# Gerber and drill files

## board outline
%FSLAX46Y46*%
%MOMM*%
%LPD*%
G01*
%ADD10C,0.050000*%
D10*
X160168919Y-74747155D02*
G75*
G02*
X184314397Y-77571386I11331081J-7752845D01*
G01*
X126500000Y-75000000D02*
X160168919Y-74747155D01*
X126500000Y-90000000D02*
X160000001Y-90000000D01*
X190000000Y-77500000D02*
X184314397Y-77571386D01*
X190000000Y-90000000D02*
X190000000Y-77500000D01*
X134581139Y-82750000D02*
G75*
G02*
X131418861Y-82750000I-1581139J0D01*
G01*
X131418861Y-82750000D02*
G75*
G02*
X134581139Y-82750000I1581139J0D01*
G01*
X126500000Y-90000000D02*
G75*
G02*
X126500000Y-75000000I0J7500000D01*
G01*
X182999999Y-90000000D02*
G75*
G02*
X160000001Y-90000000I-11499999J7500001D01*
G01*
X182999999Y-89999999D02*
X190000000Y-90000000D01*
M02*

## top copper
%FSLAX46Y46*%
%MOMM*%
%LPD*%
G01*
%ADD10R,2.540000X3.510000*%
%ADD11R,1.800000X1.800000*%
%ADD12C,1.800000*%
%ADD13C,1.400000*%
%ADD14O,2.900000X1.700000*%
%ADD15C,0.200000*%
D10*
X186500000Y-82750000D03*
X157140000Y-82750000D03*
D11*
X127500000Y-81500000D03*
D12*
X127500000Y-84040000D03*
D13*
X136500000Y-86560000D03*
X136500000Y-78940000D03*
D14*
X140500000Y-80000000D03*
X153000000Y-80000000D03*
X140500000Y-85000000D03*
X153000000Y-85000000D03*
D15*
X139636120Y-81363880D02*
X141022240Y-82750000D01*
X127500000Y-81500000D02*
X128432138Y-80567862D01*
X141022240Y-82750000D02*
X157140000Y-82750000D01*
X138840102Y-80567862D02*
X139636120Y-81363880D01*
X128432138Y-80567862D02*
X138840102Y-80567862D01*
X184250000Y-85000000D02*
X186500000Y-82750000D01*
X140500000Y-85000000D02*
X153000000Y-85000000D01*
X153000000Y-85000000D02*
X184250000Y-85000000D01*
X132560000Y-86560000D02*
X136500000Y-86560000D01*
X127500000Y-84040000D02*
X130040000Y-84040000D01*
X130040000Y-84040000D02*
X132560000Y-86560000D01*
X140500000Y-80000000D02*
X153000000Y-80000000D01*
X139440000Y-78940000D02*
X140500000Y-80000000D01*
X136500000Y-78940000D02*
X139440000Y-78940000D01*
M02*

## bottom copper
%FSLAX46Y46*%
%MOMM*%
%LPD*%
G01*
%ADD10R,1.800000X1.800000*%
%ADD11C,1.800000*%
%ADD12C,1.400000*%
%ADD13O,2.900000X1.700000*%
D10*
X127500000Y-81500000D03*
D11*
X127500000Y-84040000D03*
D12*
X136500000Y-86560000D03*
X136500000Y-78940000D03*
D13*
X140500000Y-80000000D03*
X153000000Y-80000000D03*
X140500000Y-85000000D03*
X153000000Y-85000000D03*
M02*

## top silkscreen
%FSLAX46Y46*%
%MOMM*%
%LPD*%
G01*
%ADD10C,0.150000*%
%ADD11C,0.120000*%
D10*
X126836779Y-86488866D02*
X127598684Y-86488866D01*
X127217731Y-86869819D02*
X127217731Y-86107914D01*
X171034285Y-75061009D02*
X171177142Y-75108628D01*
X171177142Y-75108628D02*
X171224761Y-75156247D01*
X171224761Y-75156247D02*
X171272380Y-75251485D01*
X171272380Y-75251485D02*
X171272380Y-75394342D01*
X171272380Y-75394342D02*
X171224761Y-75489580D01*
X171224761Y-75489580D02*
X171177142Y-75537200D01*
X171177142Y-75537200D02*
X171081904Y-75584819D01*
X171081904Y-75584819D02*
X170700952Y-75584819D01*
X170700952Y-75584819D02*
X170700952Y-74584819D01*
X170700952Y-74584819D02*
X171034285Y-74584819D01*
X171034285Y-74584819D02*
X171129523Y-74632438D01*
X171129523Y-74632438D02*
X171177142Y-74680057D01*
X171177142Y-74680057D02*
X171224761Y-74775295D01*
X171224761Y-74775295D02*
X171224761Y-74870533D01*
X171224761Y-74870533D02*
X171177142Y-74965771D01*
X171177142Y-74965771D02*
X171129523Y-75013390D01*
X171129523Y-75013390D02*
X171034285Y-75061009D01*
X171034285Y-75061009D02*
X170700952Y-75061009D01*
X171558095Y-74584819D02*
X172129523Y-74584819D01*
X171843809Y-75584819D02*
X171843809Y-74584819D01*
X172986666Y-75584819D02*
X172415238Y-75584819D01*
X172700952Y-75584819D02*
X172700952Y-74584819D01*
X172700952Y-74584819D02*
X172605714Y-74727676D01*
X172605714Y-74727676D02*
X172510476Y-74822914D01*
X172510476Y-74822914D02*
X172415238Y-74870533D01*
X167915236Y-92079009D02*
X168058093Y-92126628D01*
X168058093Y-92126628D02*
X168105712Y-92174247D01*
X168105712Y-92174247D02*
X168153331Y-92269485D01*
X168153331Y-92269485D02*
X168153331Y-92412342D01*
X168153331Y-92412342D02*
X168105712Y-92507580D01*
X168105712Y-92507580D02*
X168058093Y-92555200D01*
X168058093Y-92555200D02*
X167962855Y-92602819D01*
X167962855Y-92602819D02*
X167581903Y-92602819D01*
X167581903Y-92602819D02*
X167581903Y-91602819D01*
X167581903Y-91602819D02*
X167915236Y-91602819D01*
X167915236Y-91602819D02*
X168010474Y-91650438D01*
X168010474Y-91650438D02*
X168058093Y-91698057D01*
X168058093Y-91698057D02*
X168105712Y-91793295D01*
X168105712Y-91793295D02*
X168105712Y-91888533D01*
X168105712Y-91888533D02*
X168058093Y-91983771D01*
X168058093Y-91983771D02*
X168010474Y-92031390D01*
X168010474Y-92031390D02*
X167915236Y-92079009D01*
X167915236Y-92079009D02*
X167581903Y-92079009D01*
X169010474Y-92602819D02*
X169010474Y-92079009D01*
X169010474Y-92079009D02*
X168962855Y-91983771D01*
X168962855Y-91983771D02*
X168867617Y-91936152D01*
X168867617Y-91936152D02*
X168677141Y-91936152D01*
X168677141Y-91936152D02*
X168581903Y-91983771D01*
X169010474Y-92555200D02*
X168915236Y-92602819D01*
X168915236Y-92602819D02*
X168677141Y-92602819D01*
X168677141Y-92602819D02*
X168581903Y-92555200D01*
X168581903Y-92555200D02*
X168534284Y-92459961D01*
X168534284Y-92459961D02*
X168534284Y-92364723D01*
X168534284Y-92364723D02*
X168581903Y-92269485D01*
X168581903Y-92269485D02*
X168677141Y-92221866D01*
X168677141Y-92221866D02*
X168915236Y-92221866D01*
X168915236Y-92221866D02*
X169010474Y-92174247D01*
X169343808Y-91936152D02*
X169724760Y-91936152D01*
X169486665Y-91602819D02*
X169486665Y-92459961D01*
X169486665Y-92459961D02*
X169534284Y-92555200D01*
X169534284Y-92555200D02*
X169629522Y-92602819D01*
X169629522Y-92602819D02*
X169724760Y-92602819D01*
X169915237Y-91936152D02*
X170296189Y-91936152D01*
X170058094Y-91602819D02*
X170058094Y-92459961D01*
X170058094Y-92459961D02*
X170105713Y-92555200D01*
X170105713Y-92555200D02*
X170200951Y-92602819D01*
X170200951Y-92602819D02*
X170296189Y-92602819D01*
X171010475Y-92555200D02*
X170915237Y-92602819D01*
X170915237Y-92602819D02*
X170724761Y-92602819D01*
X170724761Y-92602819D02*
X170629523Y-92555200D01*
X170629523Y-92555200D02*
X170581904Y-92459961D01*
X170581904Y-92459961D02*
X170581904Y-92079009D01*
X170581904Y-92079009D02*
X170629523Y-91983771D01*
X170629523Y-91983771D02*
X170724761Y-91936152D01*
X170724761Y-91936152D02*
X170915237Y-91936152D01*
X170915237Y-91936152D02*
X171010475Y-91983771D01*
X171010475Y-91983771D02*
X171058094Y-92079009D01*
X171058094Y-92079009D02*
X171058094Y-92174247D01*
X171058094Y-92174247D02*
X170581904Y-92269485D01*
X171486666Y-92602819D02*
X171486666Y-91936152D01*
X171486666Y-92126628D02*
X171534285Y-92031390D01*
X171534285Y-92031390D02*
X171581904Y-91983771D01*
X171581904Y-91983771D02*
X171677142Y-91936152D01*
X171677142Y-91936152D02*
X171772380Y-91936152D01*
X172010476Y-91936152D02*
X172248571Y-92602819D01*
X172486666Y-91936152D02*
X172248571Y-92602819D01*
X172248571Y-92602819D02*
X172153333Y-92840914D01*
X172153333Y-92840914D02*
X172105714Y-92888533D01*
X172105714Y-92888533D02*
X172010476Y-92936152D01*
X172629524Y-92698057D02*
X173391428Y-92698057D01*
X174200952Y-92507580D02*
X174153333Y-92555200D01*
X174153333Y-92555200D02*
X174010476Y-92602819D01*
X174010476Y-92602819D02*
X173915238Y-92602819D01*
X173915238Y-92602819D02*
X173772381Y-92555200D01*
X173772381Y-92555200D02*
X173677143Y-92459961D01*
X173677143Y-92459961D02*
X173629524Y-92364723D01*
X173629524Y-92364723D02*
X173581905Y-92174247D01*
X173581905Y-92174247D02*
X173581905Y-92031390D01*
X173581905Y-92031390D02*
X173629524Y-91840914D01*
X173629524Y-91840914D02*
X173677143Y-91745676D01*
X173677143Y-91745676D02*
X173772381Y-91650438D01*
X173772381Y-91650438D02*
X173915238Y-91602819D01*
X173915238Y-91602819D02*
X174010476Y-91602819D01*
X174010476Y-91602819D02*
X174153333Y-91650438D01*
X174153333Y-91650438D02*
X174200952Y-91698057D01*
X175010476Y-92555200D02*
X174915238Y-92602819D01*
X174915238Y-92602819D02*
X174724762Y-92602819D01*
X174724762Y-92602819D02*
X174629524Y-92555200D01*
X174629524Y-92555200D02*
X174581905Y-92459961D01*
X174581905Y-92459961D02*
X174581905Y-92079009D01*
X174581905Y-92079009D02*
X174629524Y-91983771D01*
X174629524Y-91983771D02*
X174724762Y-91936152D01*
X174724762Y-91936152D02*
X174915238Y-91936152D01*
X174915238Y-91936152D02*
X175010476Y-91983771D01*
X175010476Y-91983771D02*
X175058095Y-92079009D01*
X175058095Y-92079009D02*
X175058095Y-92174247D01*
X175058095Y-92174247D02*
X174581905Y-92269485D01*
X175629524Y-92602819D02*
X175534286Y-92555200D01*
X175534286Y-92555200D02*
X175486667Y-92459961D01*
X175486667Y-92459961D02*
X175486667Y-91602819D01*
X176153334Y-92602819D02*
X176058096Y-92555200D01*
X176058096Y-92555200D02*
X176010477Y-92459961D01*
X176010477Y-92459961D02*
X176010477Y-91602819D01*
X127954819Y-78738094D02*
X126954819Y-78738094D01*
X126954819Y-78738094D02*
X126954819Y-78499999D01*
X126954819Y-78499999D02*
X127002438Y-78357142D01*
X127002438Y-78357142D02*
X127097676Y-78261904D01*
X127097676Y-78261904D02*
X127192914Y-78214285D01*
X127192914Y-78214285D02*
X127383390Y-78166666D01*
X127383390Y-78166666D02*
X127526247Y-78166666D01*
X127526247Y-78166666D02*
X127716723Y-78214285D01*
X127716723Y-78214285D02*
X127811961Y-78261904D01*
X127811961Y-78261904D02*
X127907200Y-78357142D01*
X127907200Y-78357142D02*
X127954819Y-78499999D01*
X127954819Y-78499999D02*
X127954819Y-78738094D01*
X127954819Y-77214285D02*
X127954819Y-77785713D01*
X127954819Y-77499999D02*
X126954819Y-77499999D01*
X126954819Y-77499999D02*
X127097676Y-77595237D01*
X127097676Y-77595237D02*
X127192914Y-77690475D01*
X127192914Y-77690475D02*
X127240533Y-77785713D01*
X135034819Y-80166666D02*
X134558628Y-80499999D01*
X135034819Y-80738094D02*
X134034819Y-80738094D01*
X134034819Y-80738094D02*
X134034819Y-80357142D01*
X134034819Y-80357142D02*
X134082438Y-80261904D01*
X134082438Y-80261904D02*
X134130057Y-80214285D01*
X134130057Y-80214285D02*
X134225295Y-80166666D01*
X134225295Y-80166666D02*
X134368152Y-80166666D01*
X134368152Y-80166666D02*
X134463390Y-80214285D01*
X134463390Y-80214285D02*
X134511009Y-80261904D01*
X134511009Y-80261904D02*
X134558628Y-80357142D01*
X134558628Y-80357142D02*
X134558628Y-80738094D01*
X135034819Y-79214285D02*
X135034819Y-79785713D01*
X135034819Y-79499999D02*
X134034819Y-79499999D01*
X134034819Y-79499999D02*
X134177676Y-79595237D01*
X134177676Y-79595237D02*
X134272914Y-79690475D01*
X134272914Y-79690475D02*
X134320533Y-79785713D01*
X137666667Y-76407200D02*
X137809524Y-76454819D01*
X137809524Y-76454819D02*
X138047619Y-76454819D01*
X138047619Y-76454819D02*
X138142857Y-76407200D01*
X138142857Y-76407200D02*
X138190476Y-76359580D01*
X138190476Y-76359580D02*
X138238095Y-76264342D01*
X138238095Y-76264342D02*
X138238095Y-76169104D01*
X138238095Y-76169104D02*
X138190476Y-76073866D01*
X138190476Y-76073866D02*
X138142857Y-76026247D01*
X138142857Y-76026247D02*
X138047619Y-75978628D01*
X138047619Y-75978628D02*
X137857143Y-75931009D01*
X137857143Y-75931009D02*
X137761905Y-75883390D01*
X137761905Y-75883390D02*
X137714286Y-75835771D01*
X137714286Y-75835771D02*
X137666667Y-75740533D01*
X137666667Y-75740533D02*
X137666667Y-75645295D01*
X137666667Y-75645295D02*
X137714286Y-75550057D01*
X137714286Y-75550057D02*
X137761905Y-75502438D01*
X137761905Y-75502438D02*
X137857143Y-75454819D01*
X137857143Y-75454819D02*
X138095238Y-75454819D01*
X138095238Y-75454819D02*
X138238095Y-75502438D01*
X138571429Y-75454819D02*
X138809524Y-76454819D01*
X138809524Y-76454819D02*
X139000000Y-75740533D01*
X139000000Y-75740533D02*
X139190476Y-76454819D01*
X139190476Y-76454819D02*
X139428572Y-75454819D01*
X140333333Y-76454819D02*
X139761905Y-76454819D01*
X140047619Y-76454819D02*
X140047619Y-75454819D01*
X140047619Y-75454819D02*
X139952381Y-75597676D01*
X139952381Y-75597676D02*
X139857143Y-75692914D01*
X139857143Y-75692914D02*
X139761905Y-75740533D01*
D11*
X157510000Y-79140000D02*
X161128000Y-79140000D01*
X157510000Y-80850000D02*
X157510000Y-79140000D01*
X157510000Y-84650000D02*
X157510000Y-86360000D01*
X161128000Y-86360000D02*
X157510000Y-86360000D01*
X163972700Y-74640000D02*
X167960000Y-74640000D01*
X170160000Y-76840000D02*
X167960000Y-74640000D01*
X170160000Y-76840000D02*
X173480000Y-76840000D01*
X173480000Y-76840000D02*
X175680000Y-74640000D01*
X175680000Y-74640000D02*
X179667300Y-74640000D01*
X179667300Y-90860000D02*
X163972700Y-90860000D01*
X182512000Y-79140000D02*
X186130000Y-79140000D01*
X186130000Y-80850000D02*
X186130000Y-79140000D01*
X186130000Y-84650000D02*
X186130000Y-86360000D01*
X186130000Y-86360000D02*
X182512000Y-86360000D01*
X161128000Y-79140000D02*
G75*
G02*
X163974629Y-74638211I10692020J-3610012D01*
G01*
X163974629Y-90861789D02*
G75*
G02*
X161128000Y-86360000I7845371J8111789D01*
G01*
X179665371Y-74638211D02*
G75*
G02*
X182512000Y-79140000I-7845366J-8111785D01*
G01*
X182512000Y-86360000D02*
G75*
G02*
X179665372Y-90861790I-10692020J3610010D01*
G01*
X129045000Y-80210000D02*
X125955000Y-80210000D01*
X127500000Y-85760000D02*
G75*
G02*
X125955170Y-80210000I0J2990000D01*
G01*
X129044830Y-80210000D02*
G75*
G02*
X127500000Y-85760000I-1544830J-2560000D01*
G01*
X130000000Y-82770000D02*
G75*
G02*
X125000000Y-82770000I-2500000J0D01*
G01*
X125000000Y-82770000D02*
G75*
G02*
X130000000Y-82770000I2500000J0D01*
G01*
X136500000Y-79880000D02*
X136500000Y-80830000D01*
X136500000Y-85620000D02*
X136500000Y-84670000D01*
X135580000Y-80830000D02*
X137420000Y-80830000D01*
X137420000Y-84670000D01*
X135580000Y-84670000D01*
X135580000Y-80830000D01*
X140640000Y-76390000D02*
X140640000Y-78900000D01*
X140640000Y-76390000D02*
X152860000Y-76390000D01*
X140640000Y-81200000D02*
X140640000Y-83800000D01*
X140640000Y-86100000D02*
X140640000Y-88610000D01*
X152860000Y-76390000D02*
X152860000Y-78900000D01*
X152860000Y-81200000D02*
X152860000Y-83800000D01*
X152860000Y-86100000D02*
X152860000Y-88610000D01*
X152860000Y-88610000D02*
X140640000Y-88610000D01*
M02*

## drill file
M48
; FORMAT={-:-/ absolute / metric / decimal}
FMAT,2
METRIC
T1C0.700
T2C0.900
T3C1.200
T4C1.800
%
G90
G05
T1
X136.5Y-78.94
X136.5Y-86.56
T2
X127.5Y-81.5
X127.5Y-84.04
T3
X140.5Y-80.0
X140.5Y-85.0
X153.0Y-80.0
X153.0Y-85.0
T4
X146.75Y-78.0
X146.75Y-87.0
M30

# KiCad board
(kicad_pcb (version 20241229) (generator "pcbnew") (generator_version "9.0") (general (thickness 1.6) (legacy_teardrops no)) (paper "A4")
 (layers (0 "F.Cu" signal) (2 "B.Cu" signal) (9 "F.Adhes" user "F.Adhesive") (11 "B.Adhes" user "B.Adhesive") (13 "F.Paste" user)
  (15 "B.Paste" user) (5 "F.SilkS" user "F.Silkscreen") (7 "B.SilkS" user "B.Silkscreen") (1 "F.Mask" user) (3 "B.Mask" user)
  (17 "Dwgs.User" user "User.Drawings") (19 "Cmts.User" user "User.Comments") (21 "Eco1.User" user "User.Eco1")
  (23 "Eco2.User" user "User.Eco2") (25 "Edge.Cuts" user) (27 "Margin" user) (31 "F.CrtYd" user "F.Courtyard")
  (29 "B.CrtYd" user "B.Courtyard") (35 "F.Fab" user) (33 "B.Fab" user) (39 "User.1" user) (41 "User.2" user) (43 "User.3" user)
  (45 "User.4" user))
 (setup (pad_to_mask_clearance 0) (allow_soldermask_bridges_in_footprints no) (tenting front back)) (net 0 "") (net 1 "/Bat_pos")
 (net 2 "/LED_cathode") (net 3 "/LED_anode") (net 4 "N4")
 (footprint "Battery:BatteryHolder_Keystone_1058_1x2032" (layer "F.Cu") (at 171.82 82.75 180)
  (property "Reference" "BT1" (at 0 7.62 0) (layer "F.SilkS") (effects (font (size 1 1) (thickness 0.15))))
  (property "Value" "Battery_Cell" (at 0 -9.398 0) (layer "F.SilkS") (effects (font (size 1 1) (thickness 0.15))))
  (fp_line (start 14.31 3.61) (end 10.692 3.61) (stroke (width 0.12) (type solid)) (layer "F.SilkS"))
  (fp_line (start 14.31 1.9) (end 14.31 3.61) (stroke (width 0.12) (type solid)) (layer "F.SilkS"))
  (fp_line (start 14.31 -1.9) (end 14.31 -3.61) (stroke (width 0.12) (type solid)) (layer "F.SilkS"))
  (fp_line (start 10.692 -3.61) (end 14.31 -3.61) (stroke (width 0.12) (type solid)) (layer "F.SilkS"))
  (fp_line (start 7.8473 8.11) (end 3.86 8.11) (stroke (width 0.12) (type solid)) (layer "F.SilkS"))
  (fp_line (start 1.66 5.91) (end 3.86 8.11) (stroke (width 0.12) (type solid)) (layer "F.SilkS"))
  (fp_line (start 1.66 5.91) (end -1.66 5.91) (stroke (width 0.12) (type solid)) (layer "F.SilkS"))
  (fp_line (start -1.66 5.91) (end -3.86 8.11) (stroke (width 0.12) (type solid)) (layer "F.SilkS"))
  (fp_line (start -3.86 8.11) (end -7.8473 8.11) (stroke (width 0.12) (type solid)) (layer "F.SilkS"))
  (fp_line (start -7.8473 -8.11) (end 7.8473 -8.11) (stroke (width 0.12) (type solid)) (layer "F.SilkS"))
  (fp_line (start -10.692 3.61) (end -14.31 3.61) (stroke (width 0.12) (type solid)) (layer "F.SilkS"))
  (fp_line (start -14.31 1.9) (end -14.31 3.61) (stroke (width 0.12) (type solid)) (layer "F.SilkS"))
  (fp_line (start -14.31 -1.9) (end -14.31 -3.61) (stroke (width 0.12) (type solid)) (layer "F.SilkS"))
  (fp_line (start -14.31 -3.61) (end -10.692 -3.61) (stroke (width 0.12) (type solid)) (layer "F.SilkS"))
  (fp_arc (start 10.692 3.61) (mid 9.538084 6.031244) (end 7.845371 8.111789) (stroke (width 0.12) (type solid)) (layer "F.SilkS"))
  (fp_arc (start 7.845371 -8.111789) (mid 9.538085 -6.031244) (end 10.692 -3.61) (stroke (width 0.12) (type solid)) (layer "F.SilkS"))
  (fp_arc (start -7.845371 8.111789) (mid -9.538085 6.031244) (end -10.692 3.61) (stroke (width 0.12) (type solid)) (layer "F.SilkS"))
  (fp_arc (start -10.692 -3.61) (mid -9.538084 -6.031244) (end -7.845371 -8.111789) (stroke (width 0.12) (type solid)) (layer "F.SilkS"))
  (pad "1" smd rect (at -14.68 0 180) (size 2.54 3.51) (layers "F.Cu" "F.Mask" "F.Paste") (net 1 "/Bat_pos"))
  (pad "2" smd rect (at 14.68 0 180) (size 2.54 3.51) (layers "F.Cu" "F.Mask" "F.Paste") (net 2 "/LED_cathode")))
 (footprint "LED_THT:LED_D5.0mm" (layer "F.Cu") (at 127.5 81.5 -90)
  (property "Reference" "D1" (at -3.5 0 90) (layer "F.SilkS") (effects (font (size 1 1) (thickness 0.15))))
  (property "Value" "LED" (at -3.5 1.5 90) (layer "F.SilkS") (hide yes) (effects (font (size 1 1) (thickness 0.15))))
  (fp_line (start -1.29 -1.545) (end -1.29 1.545) (stroke (width 0.12) (type solid)) (layer "F.SilkS"))
  (fp_arc (start 4.26 0) (mid 2.071779 2.880495) (end -1.29 1.54483) (stroke (width 0.12) (type solid)) (layer "F.SilkS"))
  (fp_arc (start -1.29 -1.54483) (mid 2.071779 -2.880495) (end 4.26 0) (stroke (width 0.12) (type solid)) (layer "F.SilkS"))
  (fp_circle (center 1.27 0) (end 3.77 0) (stroke (width 0.12) (type solid)) (fill no) (layer "F.SilkS"))
  (pad "1" thru_hole rect (at 0 0 270) (size 1.8 1.8) (drill 0.9) (layers "*.Cu" "*.Mask") (remove_unused_layers no) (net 2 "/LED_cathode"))
  (pad "2" thru_hole circle (at 2.54 0 270) (size 1.8 1.8) (drill 0.9) (layers "*.Cu" "*.Mask") (remove_unused_layers no)
   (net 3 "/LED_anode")))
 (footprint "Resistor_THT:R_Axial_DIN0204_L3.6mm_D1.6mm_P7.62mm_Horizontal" (layer "F.Cu") (at 136.5 86.56 90)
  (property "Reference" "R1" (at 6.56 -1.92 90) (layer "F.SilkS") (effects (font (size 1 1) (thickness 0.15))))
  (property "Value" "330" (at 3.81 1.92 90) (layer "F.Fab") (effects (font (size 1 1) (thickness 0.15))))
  (fp_line (start 6.68 0) (end 5.73 0) (stroke (width 0.12) (type solid)) (layer "F.SilkS"))
  (fp_line (start 0.94 0) (end 1.89 0) (stroke (width 0.12) (type solid)) (layer "F.SilkS"))
  (fp_rect (start 1.89 -0.92) (end 5.73 0.92) (stroke (width 0.12) (type solid)) (fill no) (layer "F.SilkS"))
  (pad "1" thru_hole circle (at 0 0 90) (size 1.4 1.4) (drill 0.7) (layers "*.Cu" "*.Mask") (remove_unused_layers no) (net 3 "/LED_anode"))
  (pad "2" thru_hole circle (at 7.62 0 90) (size 1.4 1.4) (drill 0.7) (layers "*.Cu" "*.Mask") (remove_unused_layers no) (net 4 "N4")))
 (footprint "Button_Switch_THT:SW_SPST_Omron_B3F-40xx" (layer "F.Cu") (at 140.5 80)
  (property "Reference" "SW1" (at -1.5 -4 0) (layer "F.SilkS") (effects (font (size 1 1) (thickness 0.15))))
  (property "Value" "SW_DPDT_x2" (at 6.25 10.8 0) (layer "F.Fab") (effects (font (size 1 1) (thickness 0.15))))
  (fp_line (start 0.14 -3.61) (end 0.14 -1.1) (stroke (width 0.12) (type default)) (layer "F.SilkS"))
  (fp_line (start 0.14 -3.61) (end 12.36 -3.61) (stroke (width 0.12) (type default)) (layer "F.SilkS"))
  (fp_line (start 0.14 1.2) (end 0.14 3.8) (stroke (width 0.12) (type default)) (layer "F.SilkS"))
  (fp_line (start 0.14 6.1) (end 0.14 8.61) (stroke (width 0.12) (type default)) (layer "F.SilkS"))
  (fp_line (start 12.36 -3.61) (end 12.36 -1.1) (stroke (width 0.12) (type default)) (layer "F.SilkS"))
  (fp_line (start 12.36 1.2) (end 12.36 3.8) (stroke (width 0.12) (type default)) (layer "F.SilkS"))
  (fp_line (start 12.36 6.1) (end 12.36 8.61) (stroke (width 0.12) (type default)) (layer "F.SilkS"))
  (fp_line (start 12.36 8.61) (end 0.14 8.61) (stroke (width 0.12) (type default)) (layer "F.SilkS"))
  (pad "" np_thru_hole circle (at 6.25 -2) (size 1.8 1.8) (drill 1.8) (layers "*.Cu" "*.Mask"))
  (pad "" np_thru_hole circle (at 6.25 7) (size 1.8 1.8) (drill 1.8) (layers "*.Cu" "*.Mask"))
  (pad "1" thru_hole oval (at 0 0) (size 2.9 1.7) (drill 1.2) (layers "*.Cu" "*.Mask") (remove_unused_layers no) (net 4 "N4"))
  (pad "1" thru_hole oval (at 12.5 0) (size 2.9 1.7) (drill 1.2) (layers "*.Cu" "*.Mask") (remove_unused_layers no) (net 4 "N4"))
  (pad "2" thru_hole oval (at 0 5) (size 2.9 1.7) (drill 1.2) (layers "*.Cu" "*.Mask") (remove_unused_layers no) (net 1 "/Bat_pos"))
  (pad "2" thru_hole oval (at 12.5 5) (size 2.9 1.7) (drill 1.2) (layers "*.Cu" "*.Mask") (remove_unused_layers no) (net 1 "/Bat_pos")))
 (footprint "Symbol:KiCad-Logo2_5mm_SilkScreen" (layer "B.Cu") (at 171.5 82.5 180)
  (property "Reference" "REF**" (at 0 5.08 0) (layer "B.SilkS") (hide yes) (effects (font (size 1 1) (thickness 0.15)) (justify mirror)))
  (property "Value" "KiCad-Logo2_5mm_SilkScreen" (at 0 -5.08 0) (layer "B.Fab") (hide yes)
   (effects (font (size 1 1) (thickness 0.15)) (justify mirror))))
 (gr_arc (start 160.168919 74.747155) (mid 173.095032 68.863436) (end 184.314397 77.571386) (stroke (width 0.05) (type default))
  (locked yes) (layer "Edge.Cuts"))
 (gr_line (start 126.5 75) (end 160.168919 74.747155) (stroke (width 0.05) (type default)) (locked yes) (layer "Edge.Cuts"))
 (gr_line (start 126.5 90) (end 160.000001 90) (stroke (width 0.05) (type default)) (locked yes) (layer "Edge.Cuts"))
 (gr_line (start 190 77.5) (end 184.314397 77.571386) (stroke (width 0.05) (type default)) (locked yes) (layer "Edge.Cuts"))
 (gr_line (start 190 90) (end 190 77.5) (stroke (width 0.05) (type default)) (locked yes) (layer "Edge.Cuts"))
 (gr_circle (center 133 82.75) (end 131.5 83.25) (stroke (width 0.05) (type default)) (fill no) (layer "Edge.Cuts"))
 (gr_arc (start 126.5 90) (mid 119 82.5) (end 126.5 75) (stroke (width 0.05) (type default)) (locked yes) (layer "Edge.Cuts"))
 (gr_arc (start 182.999999 90) (mid 171.5 96.229529) (end 160.000001 90) (stroke (width 0.05) (type default)) (locked yes)
  (layer "Edge.Cuts"))
 (gr_line (start 182.999999 89.999999) (end 190 90) (stroke (width 0.05) (type default)) (locked yes) (layer "Edge.Cuts"))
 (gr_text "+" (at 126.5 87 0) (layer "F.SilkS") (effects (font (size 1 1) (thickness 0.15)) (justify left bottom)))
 (segment (start 139.63612 81.36388) (end 141.02224 82.75) (width 0.2) (layer "F.Cu") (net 2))
 (segment (start 127.5 81.5) (end 128.432138 80.567862) (width 0.2) (layer "F.Cu") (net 2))
 (segment (start 141.02224 82.75) (end 157.14 82.75) (width 0.2) (layer "F.Cu") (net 2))
 (segment (start 138.840102 80.567862) (end 139.63612 81.36388) (width 0.2) (layer "F.Cu") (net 2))
 (segment (start 128.432138 80.567862) (end 138.840102 80.567862) (width 0.2) (layer "F.Cu") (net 2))
 (segment (start 184.25 85) (end 186.5 82.75) (width 0.2) (layer "F.Cu") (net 1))
 (segment (start 140.5 85) (end 153 85) (width 0.2) (layer "F.Cu") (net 1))
 (segment (start 153 85) (end 184.25 85) (width 0.2) (layer "F.Cu") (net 1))
 (segment (start 132.56 86.56) (end 136.5 86.56) (width 0.2) (layer "F.Cu") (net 3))
 (segment (start 127.5 84.04) (end 130.04 84.04) (width 0.2) (layer "F.Cu") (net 3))
 (segment (start 130.04 84.04) (end 132.56 86.56) (width 0.2) (layer "F.Cu") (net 3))
 (segment (start 140.5 80) (end 153 80) (width 0.2) (layer "F.Cu") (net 4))
 (segment (start 139.44 78.94) (end 140.5 80) (width 0.2) (layer "F.Cu") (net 4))
 (segment (start 136.5 78.94) (end 139.44 78.94) (width 0.2) (layer "F.Cu") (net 4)))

